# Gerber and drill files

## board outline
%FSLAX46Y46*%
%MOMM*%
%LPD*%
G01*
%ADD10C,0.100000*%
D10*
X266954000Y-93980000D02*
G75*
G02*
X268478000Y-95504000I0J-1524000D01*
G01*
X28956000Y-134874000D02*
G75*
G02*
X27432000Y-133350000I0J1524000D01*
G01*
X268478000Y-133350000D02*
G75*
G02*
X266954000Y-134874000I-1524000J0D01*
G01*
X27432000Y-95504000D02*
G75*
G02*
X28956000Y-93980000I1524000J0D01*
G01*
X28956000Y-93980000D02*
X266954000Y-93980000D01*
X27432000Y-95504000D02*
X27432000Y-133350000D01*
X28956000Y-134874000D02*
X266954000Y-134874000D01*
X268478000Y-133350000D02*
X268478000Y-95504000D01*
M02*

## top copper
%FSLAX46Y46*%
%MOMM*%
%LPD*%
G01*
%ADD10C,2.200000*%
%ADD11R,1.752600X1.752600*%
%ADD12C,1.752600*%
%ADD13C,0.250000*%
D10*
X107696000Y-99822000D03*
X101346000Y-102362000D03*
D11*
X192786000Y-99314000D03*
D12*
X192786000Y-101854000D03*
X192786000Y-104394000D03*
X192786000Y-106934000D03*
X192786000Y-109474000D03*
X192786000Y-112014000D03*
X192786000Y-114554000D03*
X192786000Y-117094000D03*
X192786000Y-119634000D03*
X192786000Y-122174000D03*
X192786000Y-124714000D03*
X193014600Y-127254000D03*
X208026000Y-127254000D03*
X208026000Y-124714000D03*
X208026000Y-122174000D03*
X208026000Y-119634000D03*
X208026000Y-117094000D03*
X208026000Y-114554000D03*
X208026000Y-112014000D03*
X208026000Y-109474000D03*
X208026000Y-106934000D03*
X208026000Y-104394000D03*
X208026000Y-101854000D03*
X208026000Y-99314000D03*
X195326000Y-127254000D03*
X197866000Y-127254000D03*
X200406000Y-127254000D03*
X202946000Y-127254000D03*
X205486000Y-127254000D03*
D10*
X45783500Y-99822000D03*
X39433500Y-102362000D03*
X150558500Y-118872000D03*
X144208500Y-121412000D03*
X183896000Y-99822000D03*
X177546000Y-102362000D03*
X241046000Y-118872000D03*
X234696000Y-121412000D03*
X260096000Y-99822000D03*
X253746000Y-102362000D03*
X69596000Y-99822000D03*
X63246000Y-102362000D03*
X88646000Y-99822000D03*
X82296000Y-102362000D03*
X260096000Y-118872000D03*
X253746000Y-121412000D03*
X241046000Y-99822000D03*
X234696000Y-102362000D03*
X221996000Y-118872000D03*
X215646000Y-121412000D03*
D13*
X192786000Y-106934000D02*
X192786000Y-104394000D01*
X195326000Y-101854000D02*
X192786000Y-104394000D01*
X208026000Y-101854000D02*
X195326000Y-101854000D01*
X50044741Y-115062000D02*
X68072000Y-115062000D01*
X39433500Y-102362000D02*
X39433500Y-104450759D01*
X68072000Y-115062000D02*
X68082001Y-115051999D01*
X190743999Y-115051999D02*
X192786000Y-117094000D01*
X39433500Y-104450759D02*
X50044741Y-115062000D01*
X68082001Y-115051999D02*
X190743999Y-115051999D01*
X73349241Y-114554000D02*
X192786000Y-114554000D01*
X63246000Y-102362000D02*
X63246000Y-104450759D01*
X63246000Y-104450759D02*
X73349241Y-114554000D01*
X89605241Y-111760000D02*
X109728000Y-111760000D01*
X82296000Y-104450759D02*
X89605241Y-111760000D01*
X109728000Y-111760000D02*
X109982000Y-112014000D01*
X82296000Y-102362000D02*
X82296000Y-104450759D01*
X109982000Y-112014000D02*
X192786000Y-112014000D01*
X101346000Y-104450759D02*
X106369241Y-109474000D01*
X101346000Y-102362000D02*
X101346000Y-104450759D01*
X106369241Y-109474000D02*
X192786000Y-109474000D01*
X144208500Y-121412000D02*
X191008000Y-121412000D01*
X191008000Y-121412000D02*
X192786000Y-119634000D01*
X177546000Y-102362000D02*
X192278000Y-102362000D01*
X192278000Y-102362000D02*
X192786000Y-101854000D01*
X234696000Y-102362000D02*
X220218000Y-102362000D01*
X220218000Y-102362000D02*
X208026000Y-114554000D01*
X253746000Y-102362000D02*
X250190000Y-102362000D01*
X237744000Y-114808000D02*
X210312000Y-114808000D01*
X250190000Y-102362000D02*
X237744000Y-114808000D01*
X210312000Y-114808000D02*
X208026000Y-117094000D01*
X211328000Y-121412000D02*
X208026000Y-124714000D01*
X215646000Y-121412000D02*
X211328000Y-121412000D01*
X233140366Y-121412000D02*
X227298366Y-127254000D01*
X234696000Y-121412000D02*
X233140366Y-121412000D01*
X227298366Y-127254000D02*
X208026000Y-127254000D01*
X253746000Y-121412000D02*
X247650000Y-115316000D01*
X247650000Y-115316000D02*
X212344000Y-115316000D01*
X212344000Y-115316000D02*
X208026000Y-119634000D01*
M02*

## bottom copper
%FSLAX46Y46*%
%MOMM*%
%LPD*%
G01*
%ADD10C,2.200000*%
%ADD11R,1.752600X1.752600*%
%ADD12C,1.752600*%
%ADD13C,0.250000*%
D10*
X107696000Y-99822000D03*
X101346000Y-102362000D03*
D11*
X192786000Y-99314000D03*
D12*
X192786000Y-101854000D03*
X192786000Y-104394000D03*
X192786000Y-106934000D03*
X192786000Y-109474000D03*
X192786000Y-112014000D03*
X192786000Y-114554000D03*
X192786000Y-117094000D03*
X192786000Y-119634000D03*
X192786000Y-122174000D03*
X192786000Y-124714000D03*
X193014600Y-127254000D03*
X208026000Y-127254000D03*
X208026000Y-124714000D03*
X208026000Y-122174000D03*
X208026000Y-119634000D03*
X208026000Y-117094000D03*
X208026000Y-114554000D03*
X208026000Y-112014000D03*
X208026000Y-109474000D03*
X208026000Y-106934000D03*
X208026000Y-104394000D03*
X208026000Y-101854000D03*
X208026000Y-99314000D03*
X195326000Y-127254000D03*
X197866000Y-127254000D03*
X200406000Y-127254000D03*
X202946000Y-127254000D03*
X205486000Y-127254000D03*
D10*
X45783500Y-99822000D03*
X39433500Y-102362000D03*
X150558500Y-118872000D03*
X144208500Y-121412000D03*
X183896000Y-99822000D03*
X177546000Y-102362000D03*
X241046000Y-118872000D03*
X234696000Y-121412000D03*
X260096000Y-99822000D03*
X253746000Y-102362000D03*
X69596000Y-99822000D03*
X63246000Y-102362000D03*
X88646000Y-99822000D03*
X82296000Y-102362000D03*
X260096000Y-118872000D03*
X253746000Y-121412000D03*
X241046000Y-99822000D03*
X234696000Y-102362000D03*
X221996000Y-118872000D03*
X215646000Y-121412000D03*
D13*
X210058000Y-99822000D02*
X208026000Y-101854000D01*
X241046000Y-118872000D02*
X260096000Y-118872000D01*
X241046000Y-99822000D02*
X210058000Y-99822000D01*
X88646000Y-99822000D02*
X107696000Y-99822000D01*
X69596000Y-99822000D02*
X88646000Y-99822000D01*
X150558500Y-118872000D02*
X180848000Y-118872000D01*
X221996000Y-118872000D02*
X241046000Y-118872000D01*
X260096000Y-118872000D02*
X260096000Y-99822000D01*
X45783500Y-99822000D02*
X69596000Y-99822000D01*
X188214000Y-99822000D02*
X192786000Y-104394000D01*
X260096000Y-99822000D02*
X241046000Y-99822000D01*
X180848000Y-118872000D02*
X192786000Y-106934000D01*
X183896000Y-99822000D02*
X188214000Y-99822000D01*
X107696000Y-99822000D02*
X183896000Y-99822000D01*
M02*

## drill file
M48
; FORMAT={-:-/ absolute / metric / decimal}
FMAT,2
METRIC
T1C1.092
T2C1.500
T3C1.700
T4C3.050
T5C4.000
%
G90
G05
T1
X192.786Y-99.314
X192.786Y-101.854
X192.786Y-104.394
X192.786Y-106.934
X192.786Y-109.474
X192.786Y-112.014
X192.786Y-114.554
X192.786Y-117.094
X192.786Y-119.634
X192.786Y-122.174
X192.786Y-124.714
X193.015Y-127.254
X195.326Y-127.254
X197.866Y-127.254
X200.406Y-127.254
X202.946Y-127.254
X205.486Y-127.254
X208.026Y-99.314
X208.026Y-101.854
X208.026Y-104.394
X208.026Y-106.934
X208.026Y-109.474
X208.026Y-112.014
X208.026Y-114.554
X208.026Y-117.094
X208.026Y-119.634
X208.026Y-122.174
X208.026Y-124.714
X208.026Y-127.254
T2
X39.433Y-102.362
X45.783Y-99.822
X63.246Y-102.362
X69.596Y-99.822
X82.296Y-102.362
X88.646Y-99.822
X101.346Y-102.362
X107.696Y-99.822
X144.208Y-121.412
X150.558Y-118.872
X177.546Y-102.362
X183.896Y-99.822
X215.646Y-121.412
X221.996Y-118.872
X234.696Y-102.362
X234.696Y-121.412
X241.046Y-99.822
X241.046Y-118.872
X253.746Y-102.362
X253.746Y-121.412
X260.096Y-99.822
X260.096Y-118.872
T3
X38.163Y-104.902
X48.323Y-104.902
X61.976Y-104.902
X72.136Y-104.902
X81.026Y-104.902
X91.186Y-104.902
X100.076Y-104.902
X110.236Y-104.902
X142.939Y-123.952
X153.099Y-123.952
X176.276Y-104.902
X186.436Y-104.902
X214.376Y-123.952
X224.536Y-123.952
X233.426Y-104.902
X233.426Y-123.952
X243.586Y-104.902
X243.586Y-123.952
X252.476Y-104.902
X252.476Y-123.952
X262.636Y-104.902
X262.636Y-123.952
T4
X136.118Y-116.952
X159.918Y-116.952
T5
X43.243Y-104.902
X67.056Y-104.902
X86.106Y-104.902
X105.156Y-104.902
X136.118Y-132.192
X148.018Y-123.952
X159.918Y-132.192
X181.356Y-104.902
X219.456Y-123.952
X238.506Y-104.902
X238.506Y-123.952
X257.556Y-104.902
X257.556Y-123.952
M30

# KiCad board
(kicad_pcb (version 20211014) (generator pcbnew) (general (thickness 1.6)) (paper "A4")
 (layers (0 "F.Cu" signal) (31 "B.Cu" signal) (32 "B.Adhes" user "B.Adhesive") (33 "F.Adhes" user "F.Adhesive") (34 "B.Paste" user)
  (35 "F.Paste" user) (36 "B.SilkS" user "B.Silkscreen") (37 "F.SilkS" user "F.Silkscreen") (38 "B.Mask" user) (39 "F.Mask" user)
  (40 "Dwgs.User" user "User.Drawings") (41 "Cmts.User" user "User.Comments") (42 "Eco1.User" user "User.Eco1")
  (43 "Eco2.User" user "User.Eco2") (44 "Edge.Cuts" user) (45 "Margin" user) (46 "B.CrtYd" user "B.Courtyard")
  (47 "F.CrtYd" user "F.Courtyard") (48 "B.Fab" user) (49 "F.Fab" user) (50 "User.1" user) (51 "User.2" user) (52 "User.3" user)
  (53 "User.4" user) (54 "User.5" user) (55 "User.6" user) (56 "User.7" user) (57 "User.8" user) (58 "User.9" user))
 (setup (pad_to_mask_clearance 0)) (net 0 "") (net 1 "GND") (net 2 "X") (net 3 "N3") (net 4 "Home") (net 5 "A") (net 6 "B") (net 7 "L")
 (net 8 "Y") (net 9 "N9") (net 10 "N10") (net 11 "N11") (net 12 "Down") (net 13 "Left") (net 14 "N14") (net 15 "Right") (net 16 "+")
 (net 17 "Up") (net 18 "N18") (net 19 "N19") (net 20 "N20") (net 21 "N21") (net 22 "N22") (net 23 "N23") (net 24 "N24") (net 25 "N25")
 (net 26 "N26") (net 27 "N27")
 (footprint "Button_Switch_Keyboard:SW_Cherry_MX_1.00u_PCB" (layer "F.Cu") (at 107.696 99.822)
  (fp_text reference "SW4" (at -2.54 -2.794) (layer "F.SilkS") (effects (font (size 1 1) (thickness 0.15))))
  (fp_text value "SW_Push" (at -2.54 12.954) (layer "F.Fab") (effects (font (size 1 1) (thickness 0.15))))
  (pad "" np_thru_hole circle (at 2.54 5.08) (size 1.7 1.7) (drill 1.7) (layers *.Cu *.Mask))
  (pad "" np_thru_hole circle (at -2.54 5.08) (size 4 4) (drill 4) (layers *.Cu *.Mask))
  (pad "" np_thru_hole circle (at -7.62 5.08) (size 1.7 1.7) (drill 1.7) (layers *.Cu *.Mask))
  (pad "1" thru_hole circle (at 0 0) (size 2.2 2.2) (drill 1.5) (layers *.Cu *.Mask) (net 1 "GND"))
  (pad "2" thru_hole circle (at -6.35 2.54) (size 2.2 2.2) (drill 1.5) (layers *.Cu *.Mask) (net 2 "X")))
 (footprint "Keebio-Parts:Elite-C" (layer "F.Cu") (at 200.406 113.284 -90)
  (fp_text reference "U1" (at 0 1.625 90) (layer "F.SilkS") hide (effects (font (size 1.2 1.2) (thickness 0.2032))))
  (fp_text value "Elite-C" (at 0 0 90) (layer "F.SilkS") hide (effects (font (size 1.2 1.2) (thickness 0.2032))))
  (pad "1" thru_hole rect locked (at -13.97 7.62 270) (size 1.7526 1.7526) (drill 1.0922) (layers *.Cu *.SilkS *.Mask) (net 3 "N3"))
  (pad "2" thru_hole circle locked (at -11.43 7.62 270) (size 1.7526 1.7526) (drill 1.0922) (layers *.Cu *.SilkS *.Mask) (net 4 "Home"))
  (pad "3" thru_hole circle locked (at -8.89 7.62 270) (size 1.7526 1.7526) (drill 1.0922) (layers *.Cu *.SilkS *.Mask) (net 1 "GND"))
  (pad "4" thru_hole circle locked (at -6.35 7.62 270) (size 1.7526 1.7526) (drill 1.0922) (layers *.Cu *.SilkS *.Mask) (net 1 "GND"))
  (pad "5" thru_hole circle locked (at -3.81 7.62 270) (size 1.7526 1.7526) (drill 1.0922) (layers *.Cu *.SilkS *.Mask) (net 2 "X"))
  (pad "6" thru_hole circle locked (at -1.27 7.62 270) (size 1.7526 1.7526) (drill 1.0922) (layers *.Cu *.SilkS *.Mask) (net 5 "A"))
  (pad "7" thru_hole circle locked (at 1.27 7.62 270) (size 1.7526 1.7526) (drill 1.0922) (layers *.Cu *.SilkS *.Mask) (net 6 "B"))
  (pad "8" thru_hole circle locked (at 3.81 7.62 270) (size 1.7526 1.7526) (drill 1.0922) (layers *.Cu *.SilkS *.Mask) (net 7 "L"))
  (pad "9" thru_hole circle locked (at 6.35 7.62 270) (size 1.7526 1.7526) (drill 1.0922) (layers *.Cu *.SilkS *.Mask) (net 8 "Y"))
  (pad "10" thru_hole circle locked (at 8.89 7.62 270) (size 1.7526 1.7526) (drill 1.0922) (layers *.Cu *.SilkS *.Mask) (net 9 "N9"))
  (pad "11" thru_hole circle locked (at 11.43 7.62 270) (size 1.7526 1.7526) (drill 1.0922) (layers *.Cu *.SilkS *.Mask) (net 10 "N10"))
  (pad "12" thru_hole circle locked (at 13.97 7.3914 270) (size 1.7526 1.7526) (drill 1.0922) (layers *.Cu *.SilkS *.Mask) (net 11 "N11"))
  (pad "13" thru_hole circle locked (at 13.97 -7.62 270) (size 1.7526 1.7526) (drill 1.0922) (layers *.Cu *.SilkS *.Mask) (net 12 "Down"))
  (pad "14" thru_hole circle locked (at 11.43 -7.62 270) (size 1.7526 1.7526) (drill 1.0922) (layers *.Cu *.SilkS *.Mask) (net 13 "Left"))
  (pad "15" thru_hole circle locked (at 8.89 -7.62 270) (size 1.7526 1.7526) (drill 1.0922) (layers *.Cu *.SilkS *.Mask) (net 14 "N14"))
  (pad "16" thru_hole circle locked (at 6.35 -7.62 270) (size 1.7526 1.7526) (drill 1.0922) (layers *.Cu *.SilkS *.Mask) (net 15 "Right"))
  (pad "17" thru_hole circle locked (at 3.81 -7.62 270) (size 1.7526 1.7526) (drill 1.0922) (layers *.Cu *.SilkS *.Mask) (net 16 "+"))
  (pad "18" thru_hole circle locked (at 1.27 -7.62 270) (size 1.7526 1.7526) (drill 1.0922) (layers *.Cu *.SilkS *.Mask) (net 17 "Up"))
  (pad "19" thru_hole circle locked (at -1.27 -7.62 270) (size 1.7526 1.7526) (drill 1.0922) (layers *.Cu *.SilkS *.Mask) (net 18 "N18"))
  (pad "20" thru_hole circle locked (at -3.81 -7.62 270) (size 1.7526 1.7526) (drill 1.0922) (layers *.Cu *.SilkS *.Mask) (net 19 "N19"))
  (pad "21" thru_hole circle locked (at -6.35 -7.62 270) (size 1.7526 1.7526) (drill 1.0922) (layers *.Cu *.SilkS *.Mask) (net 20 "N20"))
  (pad "22" thru_hole circle locked (at -8.89 -7.62 270) (size 1.7526 1.7526) (drill 1.0922) (layers *.Cu *.SilkS *.Mask) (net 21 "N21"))
  (pad "23" thru_hole circle locked (at -11.43 -7.62 270) (size 1.7526 1.7526) (drill 1.0922) (layers *.Cu *.SilkS *.Mask) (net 1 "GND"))
  (pad "24" thru_hole circle locked (at -13.97 -7.62 270) (size 1.7526 1.7526) (drill 1.0922) (layers *.Cu *.SilkS *.Mask) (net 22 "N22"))
  (pad "25" thru_hole circle locked (at 13.97 5.08 270) (size 1.7526 1.7526) (drill 1.0922) (layers *.Cu *.SilkS *.Mask) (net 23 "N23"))
  (pad "26" thru_hole circle locked (at 13.97 2.54 270) (size 1.7526 1.7526) (drill 1.0922) (layers *.Cu *.SilkS *.Mask) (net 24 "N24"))
  (pad "27" thru_hole circle locked (at 13.97 0 270) (size 1.7526 1.7526) (drill 1.0922) (layers *.Cu *.SilkS *.Mask) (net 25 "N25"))
  (pad "28" thru_hole circle locked (at 13.97 -2.54 270) (size 1.7526 1.7526) (drill 1.0922) (layers *.Cu *.SilkS *.Mask) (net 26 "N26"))
  (pad "29" thru_hole circle locked (at 13.97 -5.08 270) (size 1.7526 1.7526) (drill 1.0922) (layers *.Cu *.SilkS *.Mask) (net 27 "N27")))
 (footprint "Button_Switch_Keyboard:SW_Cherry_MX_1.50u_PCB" (layer "F.Cu") (at 45.7835 99.822)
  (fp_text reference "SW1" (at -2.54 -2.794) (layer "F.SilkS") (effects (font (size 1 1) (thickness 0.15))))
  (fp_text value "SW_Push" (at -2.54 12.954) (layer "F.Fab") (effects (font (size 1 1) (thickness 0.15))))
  (pad "" np_thru_hole circle (at -7.62 5.08) (size 1.7 1.7) (drill 1.7) (layers *.Cu *.Mask))
  (pad "" np_thru_hole circle (at 2.54 5.08) (size 1.7 1.7) (drill 1.7) (layers *.Cu *.Mask))
  (pad "" np_thru_hole circle (at -2.54 5.08) (size 4 4) (drill 4) (layers *.Cu *.Mask))
  (pad "1" thru_hole circle (at 0 0) (size 2.2 2.2) (drill 1.5) (layers *.Cu *.Mask) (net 1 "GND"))
  (pad "2" thru_hole circle (at -6.35 2.54) (size 2.2 2.2) (drill 1.5) (layers *.Cu *.Mask) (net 7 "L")))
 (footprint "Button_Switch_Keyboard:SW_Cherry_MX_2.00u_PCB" (layer "F.Cu") (at 150.5585 118.872)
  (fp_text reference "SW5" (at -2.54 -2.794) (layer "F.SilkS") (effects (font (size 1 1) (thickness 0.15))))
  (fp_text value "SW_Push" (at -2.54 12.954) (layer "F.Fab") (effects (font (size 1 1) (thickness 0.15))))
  (pad "" np_thru_hole circle (at -2.54 5.08) (size 4 4) (drill 4) (layers *.Cu *.Mask))
  (pad "" np_thru_hole circle (at -14.44 -1.92) (size 3.05 3.05) (drill 3.05) (layers *.Cu *.Mask))
  (pad "" np_thru_hole circle (at 2.54 5.08) (size 1.7 1.7) (drill 1.7) (layers *.Cu *.Mask))
  (pad "" np_thru_hole circle (at -14.44 13.32) (size 4 4) (drill 4) (layers *.Cu *.Mask))
  (pad "" np_thru_hole circle (at -7.62 5.08) (size 1.7 1.7) (drill 1.7) (layers *.Cu *.Mask))
  (pad "" np_thru_hole circle (at 9.36 13.32) (size 4 4) (drill 4) (layers *.Cu *.Mask))
  (pad "" np_thru_hole circle (at 9.36 -1.92) (size 3.05 3.05) (drill 3.05) (layers *.Cu *.Mask))
  (pad "1" thru_hole circle (at 0 0) (size 2.2 2.2) (drill 1.5) (layers *.Cu *.Mask) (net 1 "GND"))
  (pad "2" thru_hole circle (at -6.35 2.54) (size 2.2 2.2) (drill 1.5) (layers *.Cu *.Mask) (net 8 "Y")))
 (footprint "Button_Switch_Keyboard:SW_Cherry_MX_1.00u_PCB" (layer "F.Cu") (at 183.896 99.822)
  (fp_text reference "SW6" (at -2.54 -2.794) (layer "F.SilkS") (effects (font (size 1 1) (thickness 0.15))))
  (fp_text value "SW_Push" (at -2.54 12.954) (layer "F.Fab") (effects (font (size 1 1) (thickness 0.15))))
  (pad "" np_thru_hole circle (at 2.54 5.08) (size 1.7 1.7) (drill 1.7) (layers *.Cu *.Mask))
  (pad "" np_thru_hole circle (at -2.54 5.08) (size 4 4) (drill 4) (layers *.Cu *.Mask))
  (pad "" np_thru_hole circle (at -7.62 5.08) (size 1.7 1.7) (drill 1.7) (layers *.Cu *.Mask))
  (pad "1" thru_hole circle (at 0 0) (size 2.2 2.2) (drill 1.5) (layers *.Cu *.Mask) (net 1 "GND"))
  (pad "2" thru_hole circle (at -6.35 2.54) (size 2.2 2.2) (drill 1.5) (layers *.Cu *.Mask) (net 4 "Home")))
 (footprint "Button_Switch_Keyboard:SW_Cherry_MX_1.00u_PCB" (layer "F.Cu") (at 241.046 118.872)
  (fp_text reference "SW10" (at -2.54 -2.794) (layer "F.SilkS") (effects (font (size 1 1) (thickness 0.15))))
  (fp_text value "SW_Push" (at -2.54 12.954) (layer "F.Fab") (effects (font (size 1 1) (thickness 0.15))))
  (pad "" np_thru_hole circle (at -2.54 5.08) (size 4 4) (drill 4) (layers *.Cu *.Mask))
  (pad "" np_thru_hole circle (at 2.54 5.08) (size 1.7 1.7) (drill 1.7) (layers *.Cu *.Mask))
  (pad "" np_thru_hole circle (at -7.62 5.08) (size 1.7 1.7) (drill 1.7) (layers *.Cu *.Mask))
  (pad "1" thru_hole circle (at 0 0) (size 2.2 2.2) (drill 1.5) (layers *.Cu *.Mask) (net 1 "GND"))
  (pad "2" thru_hole circle (at -6.35 2.54) (size 2.2 2.2) (drill 1.5) (layers *.Cu *.Mask) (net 12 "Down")))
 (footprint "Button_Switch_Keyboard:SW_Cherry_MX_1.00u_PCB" (layer "F.Cu") (at 260.096 99.822)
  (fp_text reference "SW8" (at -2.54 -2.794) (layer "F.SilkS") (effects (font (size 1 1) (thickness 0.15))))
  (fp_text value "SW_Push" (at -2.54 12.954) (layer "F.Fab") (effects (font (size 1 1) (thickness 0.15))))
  (pad "" np_thru_hole circle (at -2.54 5.08) (size 4 4) (drill 4) (layers *.Cu *.Mask))
  (pad "" np_thru_hole circle (at 2.54 5.08) (size 1.7 1.7) (drill 1.7) (layers *.Cu *.Mask))
  (pad "" np_thru_hole circle (at -7.62 5.08) (size 1.7 1.7) (drill 1.7) (layers *.Cu *.Mask))
  (pad "1" thru_hole circle (at 0 0) (size 2.2 2.2) (drill 1.5) (layers *.Cu *.Mask) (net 1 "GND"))
  (pad "2" thru_hole circle (at -6.35 2.54) (size 2.2 2.2) (drill 1.5) (layers *.Cu *.Mask) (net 16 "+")))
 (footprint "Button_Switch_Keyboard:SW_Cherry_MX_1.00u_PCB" (layer "F.Cu") (at 69.596 99.822)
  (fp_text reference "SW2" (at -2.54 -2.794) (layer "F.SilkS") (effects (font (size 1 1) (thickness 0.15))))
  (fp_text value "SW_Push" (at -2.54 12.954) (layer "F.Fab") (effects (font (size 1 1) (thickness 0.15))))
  (pad "" np_thru_hole circle (at 2.54 5.08) (size 1.7 1.7) (drill 1.7) (layers *.Cu *.Mask))
  (pad "" np_thru_hole circle (at -7.62 5.08) (size 1.7 1.7) (drill 1.7) (layers *.Cu *.Mask))
  (pad "" np_thru_hole circle (at -2.54 5.08) (size 4 4) (drill 4) (layers *.Cu *.Mask))
  (pad "1" thru_hole circle (at 0 0) (size 2.2 2.2) (drill 1.5) (layers *.Cu *.Mask) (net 1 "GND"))
  (pad "2" thru_hole circle (at -6.35 2.54) (size 2.2 2.2) (drill 1.5) (layers *.Cu *.Mask) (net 6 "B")))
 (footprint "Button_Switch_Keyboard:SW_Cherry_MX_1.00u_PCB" (layer "F.Cu") (at 88.646 99.822)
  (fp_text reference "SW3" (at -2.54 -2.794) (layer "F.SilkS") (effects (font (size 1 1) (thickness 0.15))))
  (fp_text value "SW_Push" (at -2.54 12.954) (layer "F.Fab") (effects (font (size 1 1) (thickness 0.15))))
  (pad "" np_thru_hole circle (at 2.54 5.08) (size 1.7 1.7) (drill 1.7) (layers *.Cu *.Mask))
  (pad "" np_thru_hole circle (at -7.62 5.08) (size 1.7 1.7) (drill 1.7) (layers *.Cu *.Mask))
  (pad "" np_thru_hole circle (at -2.54 5.08) (size 4 4) (drill 4) (layers *.Cu *.Mask))
  (pad "1" thru_hole circle (at 0 0) (size 2.2 2.2) (drill 1.5) (layers *.Cu *.Mask) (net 1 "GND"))
  (pad "2" thru_hole circle (at -6.35 2.54) (size 2.2 2.2) (drill 1.5) (layers *.Cu *.Mask) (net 5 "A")))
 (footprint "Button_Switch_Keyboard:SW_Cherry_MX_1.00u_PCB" (layer "F.Cu") (at 260.096 118.872)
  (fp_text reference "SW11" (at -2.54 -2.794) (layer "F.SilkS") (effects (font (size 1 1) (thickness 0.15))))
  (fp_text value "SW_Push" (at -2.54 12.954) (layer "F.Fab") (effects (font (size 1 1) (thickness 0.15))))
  (pad "" np_thru_hole circle (at 2.54 5.08) (size 1.7 1.7) (drill 1.7) (layers *.Cu *.Mask))
  (pad "" np_thru_hole circle (at -7.62 5.08) (size 1.7 1.7) (drill 1.7) (layers *.Cu *.Mask))
  (pad "" np_thru_hole circle (at -2.54 5.08) (size 4 4) (drill 4) (layers *.Cu *.Mask))
  (pad "1" thru_hole circle (at 0 0) (size 2.2 2.2) (drill 1.5) (layers *.Cu *.Mask) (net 1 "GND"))
  (pad "2" thru_hole circle (at -6.35 2.54) (size 2.2 2.2) (drill 1.5) (layers *.Cu *.Mask) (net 15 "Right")))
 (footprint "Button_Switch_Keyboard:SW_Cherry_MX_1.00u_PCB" (layer "F.Cu") (at 241.046 99.822)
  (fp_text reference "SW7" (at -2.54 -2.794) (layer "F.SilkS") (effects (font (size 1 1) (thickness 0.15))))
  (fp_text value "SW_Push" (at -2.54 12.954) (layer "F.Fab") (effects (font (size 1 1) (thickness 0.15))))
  (pad "" np_thru_hole circle (at -2.54 5.08) (size 4 4) (drill 4) (layers *.Cu *.Mask))
  (pad "" np_thru_hole circle (at 2.54 5.08) (size 1.7 1.7) (drill 1.7) (layers *.Cu *.Mask))
  (pad "" np_thru_hole circle (at -7.62 5.08) (size 1.7 1.7) (drill 1.7) (layers *.Cu *.Mask))
  (pad "1" thru_hole circle (at 0 0) (size 2.2 2.2) (drill 1.5) (layers *.Cu *.Mask) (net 1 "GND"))
  (pad "2" thru_hole circle (at -6.35 2.54) (size 2.2 2.2) (drill 1.5) (layers *.Cu *.Mask) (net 17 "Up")))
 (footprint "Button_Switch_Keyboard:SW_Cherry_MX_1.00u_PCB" (layer "F.Cu") (at 221.996 118.872)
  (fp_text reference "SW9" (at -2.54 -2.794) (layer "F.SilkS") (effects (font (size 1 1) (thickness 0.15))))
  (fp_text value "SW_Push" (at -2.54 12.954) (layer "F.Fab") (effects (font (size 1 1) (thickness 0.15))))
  (pad "" np_thru_hole circle (at -7.62 5.08) (size 1.7 1.7) (drill 1.7) (layers *.Cu *.Mask))
  (pad "" np_thru_hole circle (at -2.54 5.08) (size 4 4) (drill 4) (layers *.Cu *.Mask))
  (pad "" np_thru_hole circle (at 2.54 5.08) (size 1.7 1.7) (drill 1.7) (layers *.Cu *.Mask))
  (pad "1" thru_hole circle (at 0 0) (size 2.2 2.2) (drill 1.5) (layers *.Cu *.Mask) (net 1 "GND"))
  (pad "2" thru_hole circle (at -6.35 2.54) (size 2.2 2.2) (drill 1.5) (layers *.Cu *.Mask) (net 13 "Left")))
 (gr_arc (start 266.954 93.98) (mid 268.031631 94.426369) (end 268.478 95.504) (layer "Edge.Cuts") (width 0.1))
 (gr_arc (start 28.956 134.874) (mid 27.878369 134.427631) (end 27.432 133.35) (layer "Edge.Cuts") (width 0.1))
 (gr_arc (start 268.478 133.35) (mid 268.031631 134.427631) (end 266.954 134.874) (layer "Edge.Cuts") (width 0.1))
 (gr_arc (start 27.432 95.504) (mid 27.878369 94.426369) (end 28.956 93.98) (layer "Edge.Cuts") (width 0.1))
 (gr_line (start 28.956 93.98) (end 266.954 93.98) (layer "Edge.Cuts") (width 0.1))
 (gr_line (start 27.432 95.504) (end 27.432 133.35) (layer "Edge.Cuts") (width 0.1))
 (gr_line (start 28.956 134.874) (end 266.954 134.874) (layer "Edge.Cuts") (width 0.1))
 (gr_line (start 268.478 133.35) (end 268.478 95.504) (layer "Edge.Cuts") (width 0.1))
 (segment (start 192.786 106.934) (end 192.786 104.394) (width 0.25) (layer "F.Cu") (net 1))
 (segment (start 195.326 101.854) (end 192.786 104.394) (width 0.25) (layer "F.Cu") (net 1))
 (segment (start 208.026 101.854) (end 195.326 101.854) (width 0.25) (layer "F.Cu") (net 1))
 (segment (start 210.058 99.822) (end 208.026 101.854) (width 0.25) (layer "B.Cu") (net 1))
 (segment (start 241.046 118.872) (end 260.096 118.872) (width 0.25) (layer "B.Cu") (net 1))
 (segment (start 241.046 99.822) (end 210.058 99.822) (width 0.25) (layer "B.Cu") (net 1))
 (segment (start 88.646 99.822) (end 107.696 99.822) (width 0.25) (layer "B.Cu") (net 1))
 (segment (start 69.596 99.822) (end 88.646 99.822) (width 0.25) (layer "B.Cu") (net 1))
 (segment (start 150.5585 118.872) (end 180.848 118.872) (width 0.25) (layer "B.Cu") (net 1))
 (segment (start 221.996 118.872) (end 241.046 118.872) (width 0.25) (layer "B.Cu") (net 1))
 (segment (start 260.096 118.872) (end 260.096 99.822) (width 0.25) (layer "B.Cu") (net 1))
 (segment (start 45.7835 99.822) (end 69.596 99.822) (width 0.25) (layer "B.Cu") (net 1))
 (segment (start 188.214 99.822) (end 192.786 104.394) (width 0.25) (layer "B.Cu") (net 1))
 (segment (start 260.096 99.822) (end 241.046 99.822) (width 0.25) (layer "B.Cu") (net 1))
 (segment (start 180.848 118.872) (end 192.786 106.934) (width 0.25) (layer "B.Cu") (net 1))
 (segment (start 183.896 99.822) (end 188.214 99.822) (width 0.25) (layer "B.Cu") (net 1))
 (segment (start 107.696 99.822) (end 183.896 99.822) (width 0.25) (layer "B.Cu") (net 1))
 (segment (start 50.044741 115.062) (end 68.072 115.062) (width 0.25) (layer "F.Cu") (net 7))
 (segment (start 39.4335 102.362) (end 39.4335 104.450759) (width 0.25) (layer "F.Cu") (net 7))
 (segment (start 68.072 115.062) (end 68.082001 115.051999) (width 0.25) (layer "F.Cu") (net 7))
 (segment (start 190.743999 115.051999) (end 192.786 117.094) (width 0.25) (layer "F.Cu") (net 7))
 (segment (start 39.4335 104.450759) (end 50.044741 115.062) (width 0.25) (layer "F.Cu") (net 7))
 (segment (start 68.082001 115.051999) (end 190.743999 115.051999) (width 0.25) (layer "F.Cu") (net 7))
 (segment (start 73.349241 114.554) (end 192.786 114.554) (width 0.25) (layer "F.Cu") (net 6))
 (segment (start 63.246 102.362) (end 63.246 104.450759) (width 0.25) (layer "F.Cu") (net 6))
 (segment (start 63.246 104.450759) (end 73.349241 114.554) (width 0.25) (layer "F.Cu") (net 6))
 (segment (start 89.605241 111.76) (end 109.728 111.76) (width 0.25) (layer "F.Cu") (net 5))
 (segment (start 82.296 104.450759) (end 89.605241 111.76) (width 0.25) (layer "F.Cu") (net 5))
 (segment (start 109.728 111.76) (end 109.982 112.014) (width 0.25) (layer "F.Cu") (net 5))
 (segment (start 82.296 102.362) (end 82.296 104.450759) (width 0.25) (layer "F.Cu") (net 5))
 (segment (start 109.982 112.014) (end 192.786 112.014) (width 0.25) (layer "F.Cu") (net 5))
 (segment (start 101.346 104.450759) (end 106.369241 109.474) (width 0.25) (layer "F.Cu") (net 2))
 (segment (start 101.346 102.362) (end 101.346 104.450759) (width 0.25) (layer "F.Cu") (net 2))
 (segment (start 106.369241 109.474) (end 192.786 109.474) (width 0.25) (layer "F.Cu") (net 2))
 (segment (start 144.2085 121.412) (end 191.008 121.412) (width 0.25) (layer "F.Cu") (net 8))
 (segment (start 191.008 121.412) (end 192.786 119.634) (width 0.25) (layer "F.Cu") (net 8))
 (segment (start 177.546 102.362) (end 192.278 102.362) (width 0.25) (layer "F.Cu") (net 4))
 (segment (start 192.278 102.362) (end 192.786 101.854) (width 0.25) (layer "F.Cu") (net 4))
 (segment (start 234.696 102.362) (end 220.218 102.362) (width 0.25) (layer "F.Cu") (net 17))
 (segment (start 220.218 102.362) (end 208.026 114.554) (width 0.25) (layer "F.Cu") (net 17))
 (segment (start 253.746 102.362) (end 250.19 102.362) (width 0.25) (layer "F.Cu") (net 16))
 (segment (start 237.744 114.808) (end 210.312 114.808) (width 0.25) (layer "F.Cu") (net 16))
 (segment (start 250.19 102.362) (end 237.744 114.808) (width 0.25) (layer "F.Cu") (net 16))
 (segment (start 210.312 114.808) (end 208.026 117.094) (width 0.25) (layer "F.Cu") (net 16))
 (segment (start 211.328 121.412) (end 208.026 124.714) (width 0.25) (layer "F.Cu") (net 13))
 (segment (start 215.646 121.412) (end 211.328 121.412) (width 0.25) (layer "F.Cu") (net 13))
 (segment (start 233.140366 121.412) (end 227.298366 127.254) (width 0.25) (layer "F.Cu") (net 12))
 (segment (start 234.696 121.412) (end 233.140366 121.412) (width 0.25) (layer "F.Cu") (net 12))
 (segment (start 227.298366 127.254) (end 208.026 127.254) (width 0.25) (layer "F.Cu") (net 12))
 (segment (start 253.746 121.412) (end 247.65 115.316) (width 0.25) (layer "F.Cu") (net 15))
 (segment (start 247.65 115.316) (end 212.344 115.316) (width 0.25) (layer "F.Cu") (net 15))
 (segment (start 212.344 115.316) (end 208.026 119.634) (width 0.25) (layer "F.Cu") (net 15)))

